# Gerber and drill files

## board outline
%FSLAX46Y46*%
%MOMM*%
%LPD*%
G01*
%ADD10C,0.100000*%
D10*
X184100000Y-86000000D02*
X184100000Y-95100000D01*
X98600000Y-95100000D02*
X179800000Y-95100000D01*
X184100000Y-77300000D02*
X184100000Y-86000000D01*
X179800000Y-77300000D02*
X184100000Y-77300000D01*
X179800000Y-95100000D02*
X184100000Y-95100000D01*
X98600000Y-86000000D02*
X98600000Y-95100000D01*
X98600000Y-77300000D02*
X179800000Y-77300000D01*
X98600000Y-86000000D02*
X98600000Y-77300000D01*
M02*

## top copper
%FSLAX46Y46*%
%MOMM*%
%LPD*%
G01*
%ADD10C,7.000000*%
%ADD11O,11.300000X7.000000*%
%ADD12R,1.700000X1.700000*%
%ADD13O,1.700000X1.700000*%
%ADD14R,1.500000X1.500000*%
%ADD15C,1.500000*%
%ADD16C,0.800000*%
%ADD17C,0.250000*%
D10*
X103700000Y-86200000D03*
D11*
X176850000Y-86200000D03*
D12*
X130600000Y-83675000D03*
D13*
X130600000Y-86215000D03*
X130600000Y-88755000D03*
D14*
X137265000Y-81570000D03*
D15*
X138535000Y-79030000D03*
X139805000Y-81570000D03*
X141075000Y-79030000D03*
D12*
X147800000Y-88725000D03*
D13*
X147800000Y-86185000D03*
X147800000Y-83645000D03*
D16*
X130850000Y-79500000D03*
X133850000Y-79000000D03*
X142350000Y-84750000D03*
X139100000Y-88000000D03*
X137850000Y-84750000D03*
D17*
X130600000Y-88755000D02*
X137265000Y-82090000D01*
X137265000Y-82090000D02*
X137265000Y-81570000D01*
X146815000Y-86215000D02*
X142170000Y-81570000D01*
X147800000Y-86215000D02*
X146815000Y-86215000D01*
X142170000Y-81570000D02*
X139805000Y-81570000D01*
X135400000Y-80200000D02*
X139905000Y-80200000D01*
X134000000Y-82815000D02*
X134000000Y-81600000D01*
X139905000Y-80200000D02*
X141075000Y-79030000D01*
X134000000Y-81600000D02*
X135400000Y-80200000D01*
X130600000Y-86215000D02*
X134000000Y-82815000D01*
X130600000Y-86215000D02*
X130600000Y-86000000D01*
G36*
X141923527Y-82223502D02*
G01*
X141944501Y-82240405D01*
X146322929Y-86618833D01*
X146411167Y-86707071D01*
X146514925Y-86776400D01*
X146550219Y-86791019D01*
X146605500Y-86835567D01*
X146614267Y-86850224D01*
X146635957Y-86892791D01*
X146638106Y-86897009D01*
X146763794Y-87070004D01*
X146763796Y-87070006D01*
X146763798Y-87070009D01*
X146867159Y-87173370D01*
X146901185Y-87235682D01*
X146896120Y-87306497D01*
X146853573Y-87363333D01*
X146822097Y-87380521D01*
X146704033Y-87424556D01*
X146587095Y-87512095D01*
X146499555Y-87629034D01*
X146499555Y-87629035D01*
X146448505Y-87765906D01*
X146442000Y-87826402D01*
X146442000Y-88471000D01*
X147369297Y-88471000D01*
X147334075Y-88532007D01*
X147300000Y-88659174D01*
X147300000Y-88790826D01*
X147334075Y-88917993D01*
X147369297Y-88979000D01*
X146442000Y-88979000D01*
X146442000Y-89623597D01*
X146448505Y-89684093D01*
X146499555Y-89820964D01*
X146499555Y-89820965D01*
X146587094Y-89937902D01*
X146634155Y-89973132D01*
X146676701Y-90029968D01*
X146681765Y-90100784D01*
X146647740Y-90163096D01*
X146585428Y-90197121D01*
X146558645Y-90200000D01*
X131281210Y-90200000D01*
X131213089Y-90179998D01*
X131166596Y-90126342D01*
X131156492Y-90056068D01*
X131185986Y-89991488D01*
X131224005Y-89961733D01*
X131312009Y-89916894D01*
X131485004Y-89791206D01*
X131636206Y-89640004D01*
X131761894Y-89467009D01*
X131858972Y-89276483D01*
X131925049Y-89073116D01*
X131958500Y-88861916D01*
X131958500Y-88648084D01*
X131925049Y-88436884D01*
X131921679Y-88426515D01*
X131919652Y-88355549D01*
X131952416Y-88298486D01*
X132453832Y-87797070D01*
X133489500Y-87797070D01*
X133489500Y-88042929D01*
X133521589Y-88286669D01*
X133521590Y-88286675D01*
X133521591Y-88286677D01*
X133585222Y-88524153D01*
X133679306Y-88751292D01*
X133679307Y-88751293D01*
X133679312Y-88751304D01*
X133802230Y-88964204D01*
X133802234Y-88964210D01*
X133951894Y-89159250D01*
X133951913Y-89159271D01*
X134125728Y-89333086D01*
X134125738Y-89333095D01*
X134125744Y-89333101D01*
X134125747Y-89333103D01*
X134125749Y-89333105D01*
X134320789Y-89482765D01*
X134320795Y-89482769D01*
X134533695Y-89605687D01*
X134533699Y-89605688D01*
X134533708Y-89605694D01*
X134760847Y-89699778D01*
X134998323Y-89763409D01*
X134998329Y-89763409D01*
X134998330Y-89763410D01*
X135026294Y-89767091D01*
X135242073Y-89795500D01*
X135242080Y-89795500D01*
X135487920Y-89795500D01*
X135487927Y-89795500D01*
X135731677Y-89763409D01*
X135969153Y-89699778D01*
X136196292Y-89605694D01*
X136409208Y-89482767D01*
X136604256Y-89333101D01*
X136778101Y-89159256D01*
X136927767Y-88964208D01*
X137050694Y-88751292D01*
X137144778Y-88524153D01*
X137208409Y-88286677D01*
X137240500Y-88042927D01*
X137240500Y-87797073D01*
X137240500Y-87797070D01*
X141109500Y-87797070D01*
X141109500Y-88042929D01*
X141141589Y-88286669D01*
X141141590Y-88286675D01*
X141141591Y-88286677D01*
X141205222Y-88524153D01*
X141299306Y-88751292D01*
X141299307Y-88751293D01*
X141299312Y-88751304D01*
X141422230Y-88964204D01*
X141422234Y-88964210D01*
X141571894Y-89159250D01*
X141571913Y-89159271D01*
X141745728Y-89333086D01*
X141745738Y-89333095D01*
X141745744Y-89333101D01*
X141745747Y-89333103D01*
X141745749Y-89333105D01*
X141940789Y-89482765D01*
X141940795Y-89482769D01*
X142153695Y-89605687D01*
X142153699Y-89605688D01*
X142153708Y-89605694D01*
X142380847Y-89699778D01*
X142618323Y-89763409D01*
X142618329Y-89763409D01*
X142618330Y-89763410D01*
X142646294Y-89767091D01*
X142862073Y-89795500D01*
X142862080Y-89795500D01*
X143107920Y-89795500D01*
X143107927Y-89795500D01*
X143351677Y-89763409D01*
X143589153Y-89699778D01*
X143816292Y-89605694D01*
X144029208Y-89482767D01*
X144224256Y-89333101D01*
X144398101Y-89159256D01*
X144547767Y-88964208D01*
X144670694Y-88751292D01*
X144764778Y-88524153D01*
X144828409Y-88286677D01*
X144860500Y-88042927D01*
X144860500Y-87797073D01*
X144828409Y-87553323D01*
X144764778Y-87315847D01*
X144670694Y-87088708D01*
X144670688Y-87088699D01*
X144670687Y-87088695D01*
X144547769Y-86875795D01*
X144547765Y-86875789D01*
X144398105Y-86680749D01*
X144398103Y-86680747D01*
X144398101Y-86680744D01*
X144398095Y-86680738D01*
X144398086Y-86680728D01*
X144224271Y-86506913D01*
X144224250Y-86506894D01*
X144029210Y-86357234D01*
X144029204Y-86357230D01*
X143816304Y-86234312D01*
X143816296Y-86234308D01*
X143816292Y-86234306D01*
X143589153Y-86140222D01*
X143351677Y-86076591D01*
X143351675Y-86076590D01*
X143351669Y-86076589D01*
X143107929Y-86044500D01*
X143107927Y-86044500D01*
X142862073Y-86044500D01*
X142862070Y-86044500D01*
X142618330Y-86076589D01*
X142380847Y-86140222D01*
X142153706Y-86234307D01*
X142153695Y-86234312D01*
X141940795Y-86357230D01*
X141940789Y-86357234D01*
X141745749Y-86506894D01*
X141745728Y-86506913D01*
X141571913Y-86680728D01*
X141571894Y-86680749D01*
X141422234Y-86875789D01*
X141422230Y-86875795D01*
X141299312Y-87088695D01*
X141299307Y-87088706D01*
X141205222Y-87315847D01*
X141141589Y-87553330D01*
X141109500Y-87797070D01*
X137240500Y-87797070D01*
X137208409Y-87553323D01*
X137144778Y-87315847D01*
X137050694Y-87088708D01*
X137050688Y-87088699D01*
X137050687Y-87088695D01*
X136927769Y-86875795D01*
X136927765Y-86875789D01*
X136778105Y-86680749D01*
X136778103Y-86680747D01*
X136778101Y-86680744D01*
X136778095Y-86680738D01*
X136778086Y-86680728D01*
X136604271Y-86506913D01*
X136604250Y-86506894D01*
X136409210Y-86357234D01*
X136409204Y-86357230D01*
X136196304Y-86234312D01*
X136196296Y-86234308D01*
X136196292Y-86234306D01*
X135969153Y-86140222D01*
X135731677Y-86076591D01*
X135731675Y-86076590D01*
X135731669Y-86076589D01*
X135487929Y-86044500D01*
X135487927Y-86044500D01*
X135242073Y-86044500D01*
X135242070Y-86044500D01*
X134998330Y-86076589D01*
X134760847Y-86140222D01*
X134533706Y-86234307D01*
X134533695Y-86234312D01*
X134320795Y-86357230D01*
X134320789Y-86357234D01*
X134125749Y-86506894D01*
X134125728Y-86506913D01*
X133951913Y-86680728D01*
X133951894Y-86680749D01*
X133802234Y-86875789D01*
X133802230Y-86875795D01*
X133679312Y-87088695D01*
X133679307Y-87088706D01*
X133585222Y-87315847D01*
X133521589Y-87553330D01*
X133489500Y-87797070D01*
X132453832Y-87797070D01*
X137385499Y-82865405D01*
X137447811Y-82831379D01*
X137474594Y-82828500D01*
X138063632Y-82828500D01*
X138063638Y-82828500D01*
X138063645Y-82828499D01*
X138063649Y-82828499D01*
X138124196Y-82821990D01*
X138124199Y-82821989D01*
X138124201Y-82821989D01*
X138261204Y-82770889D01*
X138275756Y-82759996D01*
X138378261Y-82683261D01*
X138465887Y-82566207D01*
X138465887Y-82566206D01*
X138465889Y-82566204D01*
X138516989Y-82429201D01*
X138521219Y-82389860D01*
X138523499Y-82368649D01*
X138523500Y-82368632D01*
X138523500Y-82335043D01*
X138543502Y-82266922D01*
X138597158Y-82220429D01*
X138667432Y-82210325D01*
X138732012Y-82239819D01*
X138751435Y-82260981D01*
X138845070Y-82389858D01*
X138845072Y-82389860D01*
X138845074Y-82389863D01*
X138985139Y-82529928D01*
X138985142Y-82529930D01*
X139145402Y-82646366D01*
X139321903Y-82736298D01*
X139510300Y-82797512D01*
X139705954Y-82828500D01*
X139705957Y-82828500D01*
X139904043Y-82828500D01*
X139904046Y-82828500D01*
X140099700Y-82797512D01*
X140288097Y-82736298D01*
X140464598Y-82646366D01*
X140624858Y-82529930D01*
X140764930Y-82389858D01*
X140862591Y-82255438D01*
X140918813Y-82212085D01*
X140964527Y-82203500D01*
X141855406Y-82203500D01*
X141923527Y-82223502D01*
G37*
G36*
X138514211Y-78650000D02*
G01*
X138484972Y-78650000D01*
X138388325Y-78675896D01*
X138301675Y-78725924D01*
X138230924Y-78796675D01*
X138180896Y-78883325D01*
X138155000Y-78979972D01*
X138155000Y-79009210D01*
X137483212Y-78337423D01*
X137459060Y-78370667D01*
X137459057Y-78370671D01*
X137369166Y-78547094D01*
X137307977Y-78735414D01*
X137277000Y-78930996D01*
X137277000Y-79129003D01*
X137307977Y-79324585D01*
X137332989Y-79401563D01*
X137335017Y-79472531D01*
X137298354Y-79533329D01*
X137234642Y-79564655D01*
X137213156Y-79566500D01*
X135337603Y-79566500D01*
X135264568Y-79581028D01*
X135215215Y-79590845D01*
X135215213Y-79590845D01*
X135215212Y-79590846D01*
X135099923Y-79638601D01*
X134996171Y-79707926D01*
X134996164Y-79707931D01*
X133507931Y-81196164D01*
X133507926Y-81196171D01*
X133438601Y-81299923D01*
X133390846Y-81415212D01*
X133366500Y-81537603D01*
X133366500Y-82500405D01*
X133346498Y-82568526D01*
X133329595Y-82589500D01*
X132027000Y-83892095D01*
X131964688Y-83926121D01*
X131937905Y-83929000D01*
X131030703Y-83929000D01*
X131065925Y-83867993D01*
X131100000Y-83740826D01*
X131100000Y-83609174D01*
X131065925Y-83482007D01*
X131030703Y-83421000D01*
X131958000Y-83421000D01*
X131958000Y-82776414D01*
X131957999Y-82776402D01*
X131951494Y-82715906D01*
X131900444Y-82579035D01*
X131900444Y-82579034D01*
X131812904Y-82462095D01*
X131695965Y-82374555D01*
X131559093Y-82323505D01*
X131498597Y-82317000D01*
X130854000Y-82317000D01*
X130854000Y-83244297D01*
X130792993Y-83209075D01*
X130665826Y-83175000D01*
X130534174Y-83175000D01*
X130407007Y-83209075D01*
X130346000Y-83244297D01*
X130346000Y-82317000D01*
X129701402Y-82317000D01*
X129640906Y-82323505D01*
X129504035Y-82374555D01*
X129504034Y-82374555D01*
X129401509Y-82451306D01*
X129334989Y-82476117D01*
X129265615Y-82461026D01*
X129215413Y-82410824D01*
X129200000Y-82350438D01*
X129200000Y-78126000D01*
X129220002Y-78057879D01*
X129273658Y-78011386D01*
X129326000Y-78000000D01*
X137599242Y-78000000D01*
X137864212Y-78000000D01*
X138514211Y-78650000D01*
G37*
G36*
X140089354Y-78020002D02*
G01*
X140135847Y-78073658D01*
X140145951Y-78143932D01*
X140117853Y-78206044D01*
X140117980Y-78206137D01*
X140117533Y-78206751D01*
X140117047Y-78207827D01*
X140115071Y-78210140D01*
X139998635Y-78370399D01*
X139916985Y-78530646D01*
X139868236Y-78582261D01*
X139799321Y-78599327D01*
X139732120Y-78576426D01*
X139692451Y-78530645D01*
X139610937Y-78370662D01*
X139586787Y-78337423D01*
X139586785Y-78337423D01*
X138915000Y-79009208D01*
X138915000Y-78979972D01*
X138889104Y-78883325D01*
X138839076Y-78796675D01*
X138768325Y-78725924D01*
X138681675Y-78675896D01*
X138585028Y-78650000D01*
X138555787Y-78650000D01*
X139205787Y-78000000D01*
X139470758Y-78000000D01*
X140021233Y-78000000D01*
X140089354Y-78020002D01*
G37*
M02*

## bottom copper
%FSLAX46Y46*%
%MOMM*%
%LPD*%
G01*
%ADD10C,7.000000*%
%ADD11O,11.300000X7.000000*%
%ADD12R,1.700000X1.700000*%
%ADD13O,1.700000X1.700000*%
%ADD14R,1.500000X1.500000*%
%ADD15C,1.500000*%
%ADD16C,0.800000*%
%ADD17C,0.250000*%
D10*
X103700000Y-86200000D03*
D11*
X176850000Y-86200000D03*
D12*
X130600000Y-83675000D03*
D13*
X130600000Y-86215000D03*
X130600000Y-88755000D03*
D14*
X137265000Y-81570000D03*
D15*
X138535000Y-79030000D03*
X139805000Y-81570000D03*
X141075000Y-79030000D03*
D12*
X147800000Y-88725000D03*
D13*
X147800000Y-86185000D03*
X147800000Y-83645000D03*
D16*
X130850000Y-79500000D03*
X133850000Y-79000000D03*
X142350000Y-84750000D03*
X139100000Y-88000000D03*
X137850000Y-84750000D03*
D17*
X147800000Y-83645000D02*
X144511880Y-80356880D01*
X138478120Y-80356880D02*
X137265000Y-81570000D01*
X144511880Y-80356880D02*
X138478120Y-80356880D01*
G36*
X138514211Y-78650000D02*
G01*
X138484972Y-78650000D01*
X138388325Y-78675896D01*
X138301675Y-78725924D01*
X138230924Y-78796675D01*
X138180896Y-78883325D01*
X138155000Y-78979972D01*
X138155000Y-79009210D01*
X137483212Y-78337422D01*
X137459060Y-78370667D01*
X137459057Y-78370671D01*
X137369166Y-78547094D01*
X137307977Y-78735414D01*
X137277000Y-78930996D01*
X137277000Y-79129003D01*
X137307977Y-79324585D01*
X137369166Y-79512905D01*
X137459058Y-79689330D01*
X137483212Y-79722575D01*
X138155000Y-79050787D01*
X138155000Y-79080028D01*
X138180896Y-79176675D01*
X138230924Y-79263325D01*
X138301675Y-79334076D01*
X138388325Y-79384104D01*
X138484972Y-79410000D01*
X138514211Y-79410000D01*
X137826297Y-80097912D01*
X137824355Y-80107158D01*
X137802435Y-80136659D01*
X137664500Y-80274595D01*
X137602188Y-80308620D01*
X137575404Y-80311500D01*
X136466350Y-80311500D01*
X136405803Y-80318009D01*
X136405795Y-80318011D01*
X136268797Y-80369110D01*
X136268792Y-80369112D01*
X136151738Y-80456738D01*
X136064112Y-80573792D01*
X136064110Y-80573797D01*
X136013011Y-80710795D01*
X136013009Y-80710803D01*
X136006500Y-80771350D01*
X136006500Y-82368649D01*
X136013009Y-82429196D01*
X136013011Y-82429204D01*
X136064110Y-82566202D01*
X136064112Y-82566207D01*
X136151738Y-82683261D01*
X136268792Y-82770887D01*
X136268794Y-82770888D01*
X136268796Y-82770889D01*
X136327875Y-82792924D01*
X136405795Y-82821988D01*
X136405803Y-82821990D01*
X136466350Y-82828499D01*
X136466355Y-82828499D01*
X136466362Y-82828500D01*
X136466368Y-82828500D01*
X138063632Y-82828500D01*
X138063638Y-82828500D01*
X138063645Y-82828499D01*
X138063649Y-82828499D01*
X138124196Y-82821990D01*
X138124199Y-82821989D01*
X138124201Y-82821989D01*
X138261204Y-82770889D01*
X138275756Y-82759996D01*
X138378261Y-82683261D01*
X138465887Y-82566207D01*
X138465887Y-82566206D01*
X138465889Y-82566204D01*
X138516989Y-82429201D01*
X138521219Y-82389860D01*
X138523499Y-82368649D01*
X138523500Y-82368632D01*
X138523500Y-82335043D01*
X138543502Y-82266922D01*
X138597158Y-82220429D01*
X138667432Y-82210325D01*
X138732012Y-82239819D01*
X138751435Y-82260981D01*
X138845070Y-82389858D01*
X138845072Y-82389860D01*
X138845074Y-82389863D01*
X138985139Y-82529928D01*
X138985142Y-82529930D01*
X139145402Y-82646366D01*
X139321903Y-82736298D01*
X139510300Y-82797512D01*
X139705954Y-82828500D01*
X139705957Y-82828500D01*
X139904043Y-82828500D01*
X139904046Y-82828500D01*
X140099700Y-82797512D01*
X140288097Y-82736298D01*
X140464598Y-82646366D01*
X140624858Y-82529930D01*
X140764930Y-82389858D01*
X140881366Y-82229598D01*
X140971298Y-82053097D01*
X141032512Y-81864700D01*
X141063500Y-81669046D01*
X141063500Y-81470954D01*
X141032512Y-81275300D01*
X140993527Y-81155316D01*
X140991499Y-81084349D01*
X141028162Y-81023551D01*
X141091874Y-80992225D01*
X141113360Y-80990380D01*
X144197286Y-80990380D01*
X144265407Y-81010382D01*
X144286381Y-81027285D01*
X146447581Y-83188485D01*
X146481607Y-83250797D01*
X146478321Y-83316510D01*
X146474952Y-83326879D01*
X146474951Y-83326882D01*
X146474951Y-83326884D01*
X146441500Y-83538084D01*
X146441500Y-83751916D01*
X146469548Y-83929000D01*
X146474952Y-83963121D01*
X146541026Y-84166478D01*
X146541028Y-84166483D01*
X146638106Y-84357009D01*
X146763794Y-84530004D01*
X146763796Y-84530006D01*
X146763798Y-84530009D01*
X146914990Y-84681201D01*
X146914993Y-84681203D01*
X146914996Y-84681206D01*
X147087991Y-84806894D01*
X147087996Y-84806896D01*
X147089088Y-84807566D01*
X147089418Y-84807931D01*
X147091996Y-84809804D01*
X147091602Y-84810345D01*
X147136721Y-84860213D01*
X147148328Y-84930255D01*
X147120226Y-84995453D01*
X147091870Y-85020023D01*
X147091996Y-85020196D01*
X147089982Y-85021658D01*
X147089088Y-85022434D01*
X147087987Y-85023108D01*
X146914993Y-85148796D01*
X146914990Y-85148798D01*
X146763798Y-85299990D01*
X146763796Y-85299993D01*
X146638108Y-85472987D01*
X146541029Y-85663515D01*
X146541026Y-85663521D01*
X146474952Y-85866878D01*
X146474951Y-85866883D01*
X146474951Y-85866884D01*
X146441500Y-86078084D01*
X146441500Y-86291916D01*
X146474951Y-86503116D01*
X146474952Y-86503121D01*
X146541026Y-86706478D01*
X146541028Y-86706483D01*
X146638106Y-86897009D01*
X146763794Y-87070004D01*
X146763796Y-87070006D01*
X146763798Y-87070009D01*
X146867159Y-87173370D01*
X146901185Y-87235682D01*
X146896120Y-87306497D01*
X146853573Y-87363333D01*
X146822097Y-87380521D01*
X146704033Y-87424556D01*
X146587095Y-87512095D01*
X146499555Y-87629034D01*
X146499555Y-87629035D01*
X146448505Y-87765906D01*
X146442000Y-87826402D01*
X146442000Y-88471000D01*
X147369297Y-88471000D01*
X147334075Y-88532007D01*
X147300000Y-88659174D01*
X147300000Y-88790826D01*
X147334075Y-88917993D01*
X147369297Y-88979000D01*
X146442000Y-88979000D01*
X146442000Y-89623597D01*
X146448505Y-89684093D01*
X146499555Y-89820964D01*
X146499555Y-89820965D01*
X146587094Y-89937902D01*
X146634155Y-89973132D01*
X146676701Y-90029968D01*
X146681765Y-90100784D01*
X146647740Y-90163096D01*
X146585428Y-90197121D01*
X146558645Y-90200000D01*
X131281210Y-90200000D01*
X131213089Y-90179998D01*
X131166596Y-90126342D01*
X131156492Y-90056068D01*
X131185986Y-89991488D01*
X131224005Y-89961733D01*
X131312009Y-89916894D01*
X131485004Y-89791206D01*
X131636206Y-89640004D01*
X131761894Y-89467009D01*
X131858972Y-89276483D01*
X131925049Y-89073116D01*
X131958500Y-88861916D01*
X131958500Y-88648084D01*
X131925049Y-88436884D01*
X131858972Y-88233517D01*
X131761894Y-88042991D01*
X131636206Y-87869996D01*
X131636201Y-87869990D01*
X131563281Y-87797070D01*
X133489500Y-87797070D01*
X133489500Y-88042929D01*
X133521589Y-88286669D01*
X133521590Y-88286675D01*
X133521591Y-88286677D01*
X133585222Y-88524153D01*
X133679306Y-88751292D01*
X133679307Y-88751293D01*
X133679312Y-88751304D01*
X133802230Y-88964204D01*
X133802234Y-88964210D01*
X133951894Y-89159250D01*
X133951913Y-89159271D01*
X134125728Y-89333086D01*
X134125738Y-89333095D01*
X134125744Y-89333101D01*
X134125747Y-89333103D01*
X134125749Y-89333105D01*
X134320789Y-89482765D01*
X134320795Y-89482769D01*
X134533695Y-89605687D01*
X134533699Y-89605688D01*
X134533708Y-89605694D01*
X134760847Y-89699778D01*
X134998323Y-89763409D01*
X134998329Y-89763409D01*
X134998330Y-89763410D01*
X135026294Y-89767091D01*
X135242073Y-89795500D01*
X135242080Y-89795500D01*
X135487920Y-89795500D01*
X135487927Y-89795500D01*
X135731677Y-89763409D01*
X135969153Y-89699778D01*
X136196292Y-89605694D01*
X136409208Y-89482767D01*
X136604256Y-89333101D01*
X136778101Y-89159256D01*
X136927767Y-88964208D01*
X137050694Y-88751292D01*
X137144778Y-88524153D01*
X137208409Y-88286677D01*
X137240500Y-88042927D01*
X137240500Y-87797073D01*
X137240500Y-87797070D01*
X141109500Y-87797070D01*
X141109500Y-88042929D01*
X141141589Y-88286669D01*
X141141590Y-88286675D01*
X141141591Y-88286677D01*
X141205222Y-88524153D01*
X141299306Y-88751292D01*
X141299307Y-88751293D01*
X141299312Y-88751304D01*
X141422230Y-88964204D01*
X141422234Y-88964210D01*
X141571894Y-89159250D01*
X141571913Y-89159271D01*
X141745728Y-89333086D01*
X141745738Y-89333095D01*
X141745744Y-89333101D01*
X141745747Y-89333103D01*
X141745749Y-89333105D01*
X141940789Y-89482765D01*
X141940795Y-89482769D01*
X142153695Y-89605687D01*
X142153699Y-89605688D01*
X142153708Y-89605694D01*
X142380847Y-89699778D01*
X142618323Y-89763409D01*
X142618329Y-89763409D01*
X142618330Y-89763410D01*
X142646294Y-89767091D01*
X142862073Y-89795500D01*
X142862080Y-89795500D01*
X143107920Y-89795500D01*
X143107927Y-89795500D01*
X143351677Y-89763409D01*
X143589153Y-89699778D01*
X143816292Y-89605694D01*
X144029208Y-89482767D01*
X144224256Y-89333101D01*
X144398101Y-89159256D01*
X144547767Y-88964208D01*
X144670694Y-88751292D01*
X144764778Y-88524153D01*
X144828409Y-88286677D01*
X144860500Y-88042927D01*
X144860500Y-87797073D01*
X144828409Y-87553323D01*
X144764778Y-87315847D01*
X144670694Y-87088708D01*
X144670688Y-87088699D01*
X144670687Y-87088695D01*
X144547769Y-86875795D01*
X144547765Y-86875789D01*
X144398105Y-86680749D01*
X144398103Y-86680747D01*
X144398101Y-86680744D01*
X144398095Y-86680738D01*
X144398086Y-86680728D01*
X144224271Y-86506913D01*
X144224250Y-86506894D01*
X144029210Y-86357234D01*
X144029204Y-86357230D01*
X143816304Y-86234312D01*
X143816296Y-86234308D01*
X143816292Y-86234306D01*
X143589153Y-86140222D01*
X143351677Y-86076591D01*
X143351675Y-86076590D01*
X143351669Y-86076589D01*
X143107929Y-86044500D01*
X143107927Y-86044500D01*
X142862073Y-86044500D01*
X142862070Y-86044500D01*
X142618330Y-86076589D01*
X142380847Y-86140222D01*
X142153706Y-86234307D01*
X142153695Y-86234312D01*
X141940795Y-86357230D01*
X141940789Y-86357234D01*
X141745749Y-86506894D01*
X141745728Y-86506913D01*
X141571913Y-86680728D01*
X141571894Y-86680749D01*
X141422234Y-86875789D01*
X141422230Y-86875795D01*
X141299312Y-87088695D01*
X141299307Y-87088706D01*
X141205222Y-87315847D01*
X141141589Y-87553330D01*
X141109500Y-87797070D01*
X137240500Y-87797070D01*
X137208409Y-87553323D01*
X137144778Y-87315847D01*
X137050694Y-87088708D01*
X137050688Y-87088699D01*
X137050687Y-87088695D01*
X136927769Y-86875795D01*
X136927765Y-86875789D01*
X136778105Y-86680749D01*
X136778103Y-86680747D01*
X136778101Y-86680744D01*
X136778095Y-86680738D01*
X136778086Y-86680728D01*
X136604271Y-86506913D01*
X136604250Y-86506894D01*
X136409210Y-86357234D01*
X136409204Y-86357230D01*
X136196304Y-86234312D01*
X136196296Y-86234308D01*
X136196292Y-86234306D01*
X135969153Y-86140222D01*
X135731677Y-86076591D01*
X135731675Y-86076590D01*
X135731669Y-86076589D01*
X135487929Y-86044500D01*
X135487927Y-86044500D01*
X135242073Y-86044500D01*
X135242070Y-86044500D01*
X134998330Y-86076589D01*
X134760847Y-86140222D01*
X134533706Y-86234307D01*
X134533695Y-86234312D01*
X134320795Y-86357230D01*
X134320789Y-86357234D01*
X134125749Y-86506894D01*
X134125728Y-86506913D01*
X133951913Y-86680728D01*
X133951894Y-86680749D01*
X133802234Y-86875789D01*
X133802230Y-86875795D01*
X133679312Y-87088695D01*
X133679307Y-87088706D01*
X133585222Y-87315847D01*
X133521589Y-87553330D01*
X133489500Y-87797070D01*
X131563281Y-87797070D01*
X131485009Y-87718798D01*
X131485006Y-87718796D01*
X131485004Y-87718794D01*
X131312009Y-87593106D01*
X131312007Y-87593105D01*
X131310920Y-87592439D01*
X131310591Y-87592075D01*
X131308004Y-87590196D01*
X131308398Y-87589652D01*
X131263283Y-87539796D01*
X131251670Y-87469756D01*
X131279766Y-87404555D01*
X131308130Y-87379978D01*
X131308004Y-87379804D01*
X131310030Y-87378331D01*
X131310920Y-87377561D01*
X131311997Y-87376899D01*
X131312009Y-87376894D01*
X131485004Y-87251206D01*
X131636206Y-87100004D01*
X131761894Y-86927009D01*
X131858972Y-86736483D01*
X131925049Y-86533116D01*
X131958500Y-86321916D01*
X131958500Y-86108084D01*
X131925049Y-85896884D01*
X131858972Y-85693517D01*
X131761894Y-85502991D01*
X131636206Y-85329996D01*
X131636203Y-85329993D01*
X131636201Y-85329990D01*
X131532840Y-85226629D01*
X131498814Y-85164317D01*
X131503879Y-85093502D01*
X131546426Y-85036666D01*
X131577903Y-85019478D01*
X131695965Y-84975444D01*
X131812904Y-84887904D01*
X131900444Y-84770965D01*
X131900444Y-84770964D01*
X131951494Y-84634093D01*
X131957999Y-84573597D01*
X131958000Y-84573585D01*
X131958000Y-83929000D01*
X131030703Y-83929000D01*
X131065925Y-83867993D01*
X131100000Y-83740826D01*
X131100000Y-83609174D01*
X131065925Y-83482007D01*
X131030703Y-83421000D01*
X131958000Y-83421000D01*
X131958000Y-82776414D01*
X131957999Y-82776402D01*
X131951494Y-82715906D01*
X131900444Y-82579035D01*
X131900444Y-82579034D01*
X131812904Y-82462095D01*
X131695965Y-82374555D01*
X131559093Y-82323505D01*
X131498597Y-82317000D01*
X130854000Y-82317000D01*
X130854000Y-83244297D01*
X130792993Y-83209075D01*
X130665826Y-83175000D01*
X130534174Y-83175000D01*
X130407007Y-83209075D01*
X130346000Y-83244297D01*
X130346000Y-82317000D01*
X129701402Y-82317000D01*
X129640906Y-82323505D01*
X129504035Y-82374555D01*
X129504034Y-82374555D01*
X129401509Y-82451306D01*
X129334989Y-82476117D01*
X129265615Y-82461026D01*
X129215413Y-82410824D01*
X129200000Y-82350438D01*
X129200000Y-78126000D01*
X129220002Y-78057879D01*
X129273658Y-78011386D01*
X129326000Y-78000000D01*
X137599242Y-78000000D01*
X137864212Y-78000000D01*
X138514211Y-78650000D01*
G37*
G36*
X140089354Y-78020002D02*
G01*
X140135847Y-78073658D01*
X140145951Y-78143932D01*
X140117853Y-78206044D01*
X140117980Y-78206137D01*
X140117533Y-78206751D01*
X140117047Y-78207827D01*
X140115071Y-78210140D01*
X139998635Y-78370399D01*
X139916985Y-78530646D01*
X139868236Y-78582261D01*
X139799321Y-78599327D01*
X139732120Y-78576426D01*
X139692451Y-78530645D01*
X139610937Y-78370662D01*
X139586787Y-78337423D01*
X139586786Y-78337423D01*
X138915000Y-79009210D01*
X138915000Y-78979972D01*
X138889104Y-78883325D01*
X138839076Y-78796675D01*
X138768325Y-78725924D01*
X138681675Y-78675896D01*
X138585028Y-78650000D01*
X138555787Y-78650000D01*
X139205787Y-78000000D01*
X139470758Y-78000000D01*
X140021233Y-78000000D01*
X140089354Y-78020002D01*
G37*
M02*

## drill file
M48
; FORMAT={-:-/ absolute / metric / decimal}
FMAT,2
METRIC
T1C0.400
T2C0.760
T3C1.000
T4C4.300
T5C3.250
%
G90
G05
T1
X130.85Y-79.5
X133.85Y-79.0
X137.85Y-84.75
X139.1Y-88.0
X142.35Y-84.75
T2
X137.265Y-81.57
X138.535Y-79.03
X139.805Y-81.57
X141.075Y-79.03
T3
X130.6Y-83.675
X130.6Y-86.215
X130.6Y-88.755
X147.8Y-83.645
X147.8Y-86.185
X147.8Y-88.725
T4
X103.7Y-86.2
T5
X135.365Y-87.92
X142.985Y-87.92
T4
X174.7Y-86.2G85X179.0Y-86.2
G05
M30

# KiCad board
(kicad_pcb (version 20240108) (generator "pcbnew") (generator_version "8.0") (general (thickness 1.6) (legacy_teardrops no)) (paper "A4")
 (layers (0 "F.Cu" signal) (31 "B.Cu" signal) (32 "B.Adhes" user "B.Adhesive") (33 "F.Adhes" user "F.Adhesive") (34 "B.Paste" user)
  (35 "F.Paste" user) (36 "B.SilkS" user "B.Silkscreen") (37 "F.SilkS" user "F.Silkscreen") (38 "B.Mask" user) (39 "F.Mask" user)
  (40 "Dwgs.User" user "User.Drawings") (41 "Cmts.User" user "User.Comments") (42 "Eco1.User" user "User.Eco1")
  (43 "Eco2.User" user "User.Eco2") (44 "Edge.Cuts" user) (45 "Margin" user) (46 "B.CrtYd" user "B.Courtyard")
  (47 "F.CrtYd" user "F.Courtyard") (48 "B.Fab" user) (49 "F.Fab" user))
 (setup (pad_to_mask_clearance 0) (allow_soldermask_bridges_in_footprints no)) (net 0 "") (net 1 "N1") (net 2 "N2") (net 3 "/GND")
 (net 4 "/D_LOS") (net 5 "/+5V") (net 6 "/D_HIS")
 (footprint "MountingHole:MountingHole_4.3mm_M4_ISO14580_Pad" (layer "F.Cu") (at 103.7 86.2)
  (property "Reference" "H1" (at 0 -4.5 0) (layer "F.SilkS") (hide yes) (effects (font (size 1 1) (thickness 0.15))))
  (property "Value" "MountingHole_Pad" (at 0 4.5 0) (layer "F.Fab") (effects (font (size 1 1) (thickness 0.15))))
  (pad "1" thru_hole circle (at 0 0) (size 7 7) (drill 4.3) (layers "*.Cu" "*.Mask") (remove_unused_layers no) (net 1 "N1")))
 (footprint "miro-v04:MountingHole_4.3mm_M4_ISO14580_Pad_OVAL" (layer "F.Cu") (at 176.85 86.2)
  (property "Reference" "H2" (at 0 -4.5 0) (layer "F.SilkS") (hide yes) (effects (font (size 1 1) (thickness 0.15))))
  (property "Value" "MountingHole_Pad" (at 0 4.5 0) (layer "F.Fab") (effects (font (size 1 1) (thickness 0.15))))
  (pad "1" thru_hole oval (at 0 0) (size 11.3 7) (drill oval 8.6 4.3) (layers "*.Cu" "*.Mask") (remove_unused_layers no) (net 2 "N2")))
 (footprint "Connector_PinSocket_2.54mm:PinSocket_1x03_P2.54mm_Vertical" (layer "F.Cu") (at 130.6 83.675)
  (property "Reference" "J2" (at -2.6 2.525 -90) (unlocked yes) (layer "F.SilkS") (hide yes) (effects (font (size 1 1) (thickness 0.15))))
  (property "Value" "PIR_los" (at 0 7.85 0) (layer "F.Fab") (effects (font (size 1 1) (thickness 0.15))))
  (pad "1" thru_hole rect (at 0 0) (size 1.7 1.7) (drill 1) (layers "*.Cu" "*.Mask") (remove_unused_layers no) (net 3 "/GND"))
  (pad "2" thru_hole oval (at 0 2.54) (size 1.7 1.7) (drill 1) (layers "*.Cu" "*.Mask") (remove_unused_layers no) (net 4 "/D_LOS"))
  (pad "3" thru_hole oval (at 0 5.08) (size 1.7 1.7) (drill 1) (layers "*.Cu" "*.Mask") (remove_unused_layers no) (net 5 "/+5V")))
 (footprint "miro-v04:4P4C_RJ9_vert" (layer "F.Cu") (at 137.265 81.57 180)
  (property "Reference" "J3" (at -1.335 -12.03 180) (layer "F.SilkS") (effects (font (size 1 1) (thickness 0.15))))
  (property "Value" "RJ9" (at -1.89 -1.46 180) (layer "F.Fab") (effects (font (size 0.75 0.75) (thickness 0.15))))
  (pad "" np_thru_hole circle (at -5.72 -6.35 180) (size 3.25 3.25) (drill 3.25) (layers "*.Cu" "*.Mask"))
  (pad "" np_thru_hole circle (at 1.9 -6.35 180) (size 3.25 3.25) (drill 3.25) (layers "*.Cu" "*.Mask"))
  (pad "1" thru_hole rect (at 0 0) (size 1.5 1.5) (drill 0.76) (layers "*.Cu" "*.Mask") (remove_unused_layers no) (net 5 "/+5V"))
  (pad "2" thru_hole circle (at -1.27 2.54) (size 1.5 1.5) (drill 0.76) (layers "*.Cu" "*.Mask") (remove_unused_layers no) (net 3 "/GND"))
  (pad "3" thru_hole circle (at -2.54 0) (size 1.5 1.5) (drill 0.76) (layers "*.Cu" "*.Mask") (remove_unused_layers no) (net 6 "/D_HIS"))
  (pad "4" thru_hole circle (at -3.81 2.54) (size 1.5 1.5) (drill 0.76) (layers "*.Cu" "*.Mask") (remove_unused_layers no) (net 4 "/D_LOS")))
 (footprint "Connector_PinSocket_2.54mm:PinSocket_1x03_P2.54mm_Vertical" (layer "F.Cu") (at 147.8 88.725 180)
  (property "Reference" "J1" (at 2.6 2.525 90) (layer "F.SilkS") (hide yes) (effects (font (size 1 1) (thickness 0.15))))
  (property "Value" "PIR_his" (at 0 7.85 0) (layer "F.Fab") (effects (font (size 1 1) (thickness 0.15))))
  (pad "1" thru_hole rect (at 0 0 180) (size 1.7 1.7) (drill 1) (layers "*.Cu" "*.Mask") (remove_unused_layers no) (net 3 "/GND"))
  (pad "2" thru_hole oval (at 0 2.54 180) (size 1.7 1.7) (drill 1) (layers "*.Cu" "*.Mask") (remove_unused_layers no) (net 6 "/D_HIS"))
  (pad "3" thru_hole oval (at 0 5.08 180) (size 1.7 1.7) (drill 1) (layers "*.Cu" "*.Mask") (remove_unused_layers no) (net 5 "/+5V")))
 (gr_line (start 184.1 86) (end 184.1 95.1) (stroke (width 0.1) (type solid)) (layer "Edge.Cuts"))
 (gr_line (start 98.6 95.1) (end 179.8 95.1) (stroke (width 0.1) (type solid)) (layer "Edge.Cuts"))
 (gr_line (start 184.1 77.3) (end 184.1 86) (stroke (width 0.1) (type solid)) (layer "Edge.Cuts"))
 (gr_line (start 179.8 77.3) (end 184.1 77.3) (stroke (width 0.1) (type solid)) (layer "Edge.Cuts"))
 (gr_line (start 179.8 95.1) (end 184.1 95.1) (stroke (width 0.1) (type solid)) (layer "Edge.Cuts"))
 (gr_line (start 98.6 86) (end 98.6 95.1) (stroke (width 0.1) (type solid)) (layer "Edge.Cuts"))
 (gr_line (start 98.6 77.3) (end 179.8 77.3) (stroke (width 0.1) (type solid)) (layer "Edge.Cuts"))
 (gr_line (start 98.6 86) (end 98.6 77.3) (stroke (width 0.1) (type solid)) (layer "Edge.Cuts"))
 (segment (start 130.6 88.755) (end 137.265 82.09) (width 0.25) (layer "F.Cu") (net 5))
 (segment (start 137.265 82.09) (end 137.265 81.57) (width 0.25) (layer "F.Cu") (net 5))
 (segment (start 147.8 83.645) (end 144.51188 80.35688) (width 0.25) (layer "B.Cu") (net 5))
 (segment (start 138.47812 80.35688) (end 137.265 81.57) (width 0.25) (layer "B.Cu") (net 5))
 (segment (start 144.51188 80.35688) (end 138.47812 80.35688) (width 0.25) (layer "B.Cu") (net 5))
 (segment (start 146.815 86.215) (end 142.17 81.57) (width 0.25) (layer "F.Cu") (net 6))
 (segment (start 147.8 86.215) (end 146.815 86.215) (width 0.25) (layer "F.Cu") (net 6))
 (segment (start 142.17 81.57) (end 139.805 81.57) (width 0.25) (layer "F.Cu") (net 6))
 (via (at 130.85 79.5) (size 0.8) (drill 0.4) (layers "F.Cu" "B.Cu") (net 3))
 (via (at 133.85 79) (size 0.8) (drill 0.4) (layers "F.Cu" "B.Cu") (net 3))
 (via (at 142.35 84.75) (size 0.8) (drill 0.4) (layers "F.Cu" "B.Cu") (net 3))
 (via (at 139.1 88) (size 0.8) (drill 0.4) (layers "F.Cu" "B.Cu") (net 3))
 (via (at 137.85 84.75) (size 0.8) (drill 0.4) (layers "F.Cu" "B.Cu") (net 3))
 (segment (start 135.4 80.2) (end 139.905 80.2) (width 0.25) (layer "F.Cu") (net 4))
 (segment (start 134 82.815) (end 134 81.6) (width 0.25) (layer "F.Cu") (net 4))
 (segment (start 139.905 80.2) (end 141.075 79.03) (width 0.25) (layer "F.Cu") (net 4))
 (segment (start 134 81.6) (end 135.4 80.2) (width 0.25) (layer "F.Cu") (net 4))
 (segment (start 130.6 86.215) (end 134 82.815) (width 0.25) (layer "F.Cu") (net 4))
 (segment (start 130.6 86.215) (end 130.6 86) (width 0.25) (layer "F.Cu") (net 4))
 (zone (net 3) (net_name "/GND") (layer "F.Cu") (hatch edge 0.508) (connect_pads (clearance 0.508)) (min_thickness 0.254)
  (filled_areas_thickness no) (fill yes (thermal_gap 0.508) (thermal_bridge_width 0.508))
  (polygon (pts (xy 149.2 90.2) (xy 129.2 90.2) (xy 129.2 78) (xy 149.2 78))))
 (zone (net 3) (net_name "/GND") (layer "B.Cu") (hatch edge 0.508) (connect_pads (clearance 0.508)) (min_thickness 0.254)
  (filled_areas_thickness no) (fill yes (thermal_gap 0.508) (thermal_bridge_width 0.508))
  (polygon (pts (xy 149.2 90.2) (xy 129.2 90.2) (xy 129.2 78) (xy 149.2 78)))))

